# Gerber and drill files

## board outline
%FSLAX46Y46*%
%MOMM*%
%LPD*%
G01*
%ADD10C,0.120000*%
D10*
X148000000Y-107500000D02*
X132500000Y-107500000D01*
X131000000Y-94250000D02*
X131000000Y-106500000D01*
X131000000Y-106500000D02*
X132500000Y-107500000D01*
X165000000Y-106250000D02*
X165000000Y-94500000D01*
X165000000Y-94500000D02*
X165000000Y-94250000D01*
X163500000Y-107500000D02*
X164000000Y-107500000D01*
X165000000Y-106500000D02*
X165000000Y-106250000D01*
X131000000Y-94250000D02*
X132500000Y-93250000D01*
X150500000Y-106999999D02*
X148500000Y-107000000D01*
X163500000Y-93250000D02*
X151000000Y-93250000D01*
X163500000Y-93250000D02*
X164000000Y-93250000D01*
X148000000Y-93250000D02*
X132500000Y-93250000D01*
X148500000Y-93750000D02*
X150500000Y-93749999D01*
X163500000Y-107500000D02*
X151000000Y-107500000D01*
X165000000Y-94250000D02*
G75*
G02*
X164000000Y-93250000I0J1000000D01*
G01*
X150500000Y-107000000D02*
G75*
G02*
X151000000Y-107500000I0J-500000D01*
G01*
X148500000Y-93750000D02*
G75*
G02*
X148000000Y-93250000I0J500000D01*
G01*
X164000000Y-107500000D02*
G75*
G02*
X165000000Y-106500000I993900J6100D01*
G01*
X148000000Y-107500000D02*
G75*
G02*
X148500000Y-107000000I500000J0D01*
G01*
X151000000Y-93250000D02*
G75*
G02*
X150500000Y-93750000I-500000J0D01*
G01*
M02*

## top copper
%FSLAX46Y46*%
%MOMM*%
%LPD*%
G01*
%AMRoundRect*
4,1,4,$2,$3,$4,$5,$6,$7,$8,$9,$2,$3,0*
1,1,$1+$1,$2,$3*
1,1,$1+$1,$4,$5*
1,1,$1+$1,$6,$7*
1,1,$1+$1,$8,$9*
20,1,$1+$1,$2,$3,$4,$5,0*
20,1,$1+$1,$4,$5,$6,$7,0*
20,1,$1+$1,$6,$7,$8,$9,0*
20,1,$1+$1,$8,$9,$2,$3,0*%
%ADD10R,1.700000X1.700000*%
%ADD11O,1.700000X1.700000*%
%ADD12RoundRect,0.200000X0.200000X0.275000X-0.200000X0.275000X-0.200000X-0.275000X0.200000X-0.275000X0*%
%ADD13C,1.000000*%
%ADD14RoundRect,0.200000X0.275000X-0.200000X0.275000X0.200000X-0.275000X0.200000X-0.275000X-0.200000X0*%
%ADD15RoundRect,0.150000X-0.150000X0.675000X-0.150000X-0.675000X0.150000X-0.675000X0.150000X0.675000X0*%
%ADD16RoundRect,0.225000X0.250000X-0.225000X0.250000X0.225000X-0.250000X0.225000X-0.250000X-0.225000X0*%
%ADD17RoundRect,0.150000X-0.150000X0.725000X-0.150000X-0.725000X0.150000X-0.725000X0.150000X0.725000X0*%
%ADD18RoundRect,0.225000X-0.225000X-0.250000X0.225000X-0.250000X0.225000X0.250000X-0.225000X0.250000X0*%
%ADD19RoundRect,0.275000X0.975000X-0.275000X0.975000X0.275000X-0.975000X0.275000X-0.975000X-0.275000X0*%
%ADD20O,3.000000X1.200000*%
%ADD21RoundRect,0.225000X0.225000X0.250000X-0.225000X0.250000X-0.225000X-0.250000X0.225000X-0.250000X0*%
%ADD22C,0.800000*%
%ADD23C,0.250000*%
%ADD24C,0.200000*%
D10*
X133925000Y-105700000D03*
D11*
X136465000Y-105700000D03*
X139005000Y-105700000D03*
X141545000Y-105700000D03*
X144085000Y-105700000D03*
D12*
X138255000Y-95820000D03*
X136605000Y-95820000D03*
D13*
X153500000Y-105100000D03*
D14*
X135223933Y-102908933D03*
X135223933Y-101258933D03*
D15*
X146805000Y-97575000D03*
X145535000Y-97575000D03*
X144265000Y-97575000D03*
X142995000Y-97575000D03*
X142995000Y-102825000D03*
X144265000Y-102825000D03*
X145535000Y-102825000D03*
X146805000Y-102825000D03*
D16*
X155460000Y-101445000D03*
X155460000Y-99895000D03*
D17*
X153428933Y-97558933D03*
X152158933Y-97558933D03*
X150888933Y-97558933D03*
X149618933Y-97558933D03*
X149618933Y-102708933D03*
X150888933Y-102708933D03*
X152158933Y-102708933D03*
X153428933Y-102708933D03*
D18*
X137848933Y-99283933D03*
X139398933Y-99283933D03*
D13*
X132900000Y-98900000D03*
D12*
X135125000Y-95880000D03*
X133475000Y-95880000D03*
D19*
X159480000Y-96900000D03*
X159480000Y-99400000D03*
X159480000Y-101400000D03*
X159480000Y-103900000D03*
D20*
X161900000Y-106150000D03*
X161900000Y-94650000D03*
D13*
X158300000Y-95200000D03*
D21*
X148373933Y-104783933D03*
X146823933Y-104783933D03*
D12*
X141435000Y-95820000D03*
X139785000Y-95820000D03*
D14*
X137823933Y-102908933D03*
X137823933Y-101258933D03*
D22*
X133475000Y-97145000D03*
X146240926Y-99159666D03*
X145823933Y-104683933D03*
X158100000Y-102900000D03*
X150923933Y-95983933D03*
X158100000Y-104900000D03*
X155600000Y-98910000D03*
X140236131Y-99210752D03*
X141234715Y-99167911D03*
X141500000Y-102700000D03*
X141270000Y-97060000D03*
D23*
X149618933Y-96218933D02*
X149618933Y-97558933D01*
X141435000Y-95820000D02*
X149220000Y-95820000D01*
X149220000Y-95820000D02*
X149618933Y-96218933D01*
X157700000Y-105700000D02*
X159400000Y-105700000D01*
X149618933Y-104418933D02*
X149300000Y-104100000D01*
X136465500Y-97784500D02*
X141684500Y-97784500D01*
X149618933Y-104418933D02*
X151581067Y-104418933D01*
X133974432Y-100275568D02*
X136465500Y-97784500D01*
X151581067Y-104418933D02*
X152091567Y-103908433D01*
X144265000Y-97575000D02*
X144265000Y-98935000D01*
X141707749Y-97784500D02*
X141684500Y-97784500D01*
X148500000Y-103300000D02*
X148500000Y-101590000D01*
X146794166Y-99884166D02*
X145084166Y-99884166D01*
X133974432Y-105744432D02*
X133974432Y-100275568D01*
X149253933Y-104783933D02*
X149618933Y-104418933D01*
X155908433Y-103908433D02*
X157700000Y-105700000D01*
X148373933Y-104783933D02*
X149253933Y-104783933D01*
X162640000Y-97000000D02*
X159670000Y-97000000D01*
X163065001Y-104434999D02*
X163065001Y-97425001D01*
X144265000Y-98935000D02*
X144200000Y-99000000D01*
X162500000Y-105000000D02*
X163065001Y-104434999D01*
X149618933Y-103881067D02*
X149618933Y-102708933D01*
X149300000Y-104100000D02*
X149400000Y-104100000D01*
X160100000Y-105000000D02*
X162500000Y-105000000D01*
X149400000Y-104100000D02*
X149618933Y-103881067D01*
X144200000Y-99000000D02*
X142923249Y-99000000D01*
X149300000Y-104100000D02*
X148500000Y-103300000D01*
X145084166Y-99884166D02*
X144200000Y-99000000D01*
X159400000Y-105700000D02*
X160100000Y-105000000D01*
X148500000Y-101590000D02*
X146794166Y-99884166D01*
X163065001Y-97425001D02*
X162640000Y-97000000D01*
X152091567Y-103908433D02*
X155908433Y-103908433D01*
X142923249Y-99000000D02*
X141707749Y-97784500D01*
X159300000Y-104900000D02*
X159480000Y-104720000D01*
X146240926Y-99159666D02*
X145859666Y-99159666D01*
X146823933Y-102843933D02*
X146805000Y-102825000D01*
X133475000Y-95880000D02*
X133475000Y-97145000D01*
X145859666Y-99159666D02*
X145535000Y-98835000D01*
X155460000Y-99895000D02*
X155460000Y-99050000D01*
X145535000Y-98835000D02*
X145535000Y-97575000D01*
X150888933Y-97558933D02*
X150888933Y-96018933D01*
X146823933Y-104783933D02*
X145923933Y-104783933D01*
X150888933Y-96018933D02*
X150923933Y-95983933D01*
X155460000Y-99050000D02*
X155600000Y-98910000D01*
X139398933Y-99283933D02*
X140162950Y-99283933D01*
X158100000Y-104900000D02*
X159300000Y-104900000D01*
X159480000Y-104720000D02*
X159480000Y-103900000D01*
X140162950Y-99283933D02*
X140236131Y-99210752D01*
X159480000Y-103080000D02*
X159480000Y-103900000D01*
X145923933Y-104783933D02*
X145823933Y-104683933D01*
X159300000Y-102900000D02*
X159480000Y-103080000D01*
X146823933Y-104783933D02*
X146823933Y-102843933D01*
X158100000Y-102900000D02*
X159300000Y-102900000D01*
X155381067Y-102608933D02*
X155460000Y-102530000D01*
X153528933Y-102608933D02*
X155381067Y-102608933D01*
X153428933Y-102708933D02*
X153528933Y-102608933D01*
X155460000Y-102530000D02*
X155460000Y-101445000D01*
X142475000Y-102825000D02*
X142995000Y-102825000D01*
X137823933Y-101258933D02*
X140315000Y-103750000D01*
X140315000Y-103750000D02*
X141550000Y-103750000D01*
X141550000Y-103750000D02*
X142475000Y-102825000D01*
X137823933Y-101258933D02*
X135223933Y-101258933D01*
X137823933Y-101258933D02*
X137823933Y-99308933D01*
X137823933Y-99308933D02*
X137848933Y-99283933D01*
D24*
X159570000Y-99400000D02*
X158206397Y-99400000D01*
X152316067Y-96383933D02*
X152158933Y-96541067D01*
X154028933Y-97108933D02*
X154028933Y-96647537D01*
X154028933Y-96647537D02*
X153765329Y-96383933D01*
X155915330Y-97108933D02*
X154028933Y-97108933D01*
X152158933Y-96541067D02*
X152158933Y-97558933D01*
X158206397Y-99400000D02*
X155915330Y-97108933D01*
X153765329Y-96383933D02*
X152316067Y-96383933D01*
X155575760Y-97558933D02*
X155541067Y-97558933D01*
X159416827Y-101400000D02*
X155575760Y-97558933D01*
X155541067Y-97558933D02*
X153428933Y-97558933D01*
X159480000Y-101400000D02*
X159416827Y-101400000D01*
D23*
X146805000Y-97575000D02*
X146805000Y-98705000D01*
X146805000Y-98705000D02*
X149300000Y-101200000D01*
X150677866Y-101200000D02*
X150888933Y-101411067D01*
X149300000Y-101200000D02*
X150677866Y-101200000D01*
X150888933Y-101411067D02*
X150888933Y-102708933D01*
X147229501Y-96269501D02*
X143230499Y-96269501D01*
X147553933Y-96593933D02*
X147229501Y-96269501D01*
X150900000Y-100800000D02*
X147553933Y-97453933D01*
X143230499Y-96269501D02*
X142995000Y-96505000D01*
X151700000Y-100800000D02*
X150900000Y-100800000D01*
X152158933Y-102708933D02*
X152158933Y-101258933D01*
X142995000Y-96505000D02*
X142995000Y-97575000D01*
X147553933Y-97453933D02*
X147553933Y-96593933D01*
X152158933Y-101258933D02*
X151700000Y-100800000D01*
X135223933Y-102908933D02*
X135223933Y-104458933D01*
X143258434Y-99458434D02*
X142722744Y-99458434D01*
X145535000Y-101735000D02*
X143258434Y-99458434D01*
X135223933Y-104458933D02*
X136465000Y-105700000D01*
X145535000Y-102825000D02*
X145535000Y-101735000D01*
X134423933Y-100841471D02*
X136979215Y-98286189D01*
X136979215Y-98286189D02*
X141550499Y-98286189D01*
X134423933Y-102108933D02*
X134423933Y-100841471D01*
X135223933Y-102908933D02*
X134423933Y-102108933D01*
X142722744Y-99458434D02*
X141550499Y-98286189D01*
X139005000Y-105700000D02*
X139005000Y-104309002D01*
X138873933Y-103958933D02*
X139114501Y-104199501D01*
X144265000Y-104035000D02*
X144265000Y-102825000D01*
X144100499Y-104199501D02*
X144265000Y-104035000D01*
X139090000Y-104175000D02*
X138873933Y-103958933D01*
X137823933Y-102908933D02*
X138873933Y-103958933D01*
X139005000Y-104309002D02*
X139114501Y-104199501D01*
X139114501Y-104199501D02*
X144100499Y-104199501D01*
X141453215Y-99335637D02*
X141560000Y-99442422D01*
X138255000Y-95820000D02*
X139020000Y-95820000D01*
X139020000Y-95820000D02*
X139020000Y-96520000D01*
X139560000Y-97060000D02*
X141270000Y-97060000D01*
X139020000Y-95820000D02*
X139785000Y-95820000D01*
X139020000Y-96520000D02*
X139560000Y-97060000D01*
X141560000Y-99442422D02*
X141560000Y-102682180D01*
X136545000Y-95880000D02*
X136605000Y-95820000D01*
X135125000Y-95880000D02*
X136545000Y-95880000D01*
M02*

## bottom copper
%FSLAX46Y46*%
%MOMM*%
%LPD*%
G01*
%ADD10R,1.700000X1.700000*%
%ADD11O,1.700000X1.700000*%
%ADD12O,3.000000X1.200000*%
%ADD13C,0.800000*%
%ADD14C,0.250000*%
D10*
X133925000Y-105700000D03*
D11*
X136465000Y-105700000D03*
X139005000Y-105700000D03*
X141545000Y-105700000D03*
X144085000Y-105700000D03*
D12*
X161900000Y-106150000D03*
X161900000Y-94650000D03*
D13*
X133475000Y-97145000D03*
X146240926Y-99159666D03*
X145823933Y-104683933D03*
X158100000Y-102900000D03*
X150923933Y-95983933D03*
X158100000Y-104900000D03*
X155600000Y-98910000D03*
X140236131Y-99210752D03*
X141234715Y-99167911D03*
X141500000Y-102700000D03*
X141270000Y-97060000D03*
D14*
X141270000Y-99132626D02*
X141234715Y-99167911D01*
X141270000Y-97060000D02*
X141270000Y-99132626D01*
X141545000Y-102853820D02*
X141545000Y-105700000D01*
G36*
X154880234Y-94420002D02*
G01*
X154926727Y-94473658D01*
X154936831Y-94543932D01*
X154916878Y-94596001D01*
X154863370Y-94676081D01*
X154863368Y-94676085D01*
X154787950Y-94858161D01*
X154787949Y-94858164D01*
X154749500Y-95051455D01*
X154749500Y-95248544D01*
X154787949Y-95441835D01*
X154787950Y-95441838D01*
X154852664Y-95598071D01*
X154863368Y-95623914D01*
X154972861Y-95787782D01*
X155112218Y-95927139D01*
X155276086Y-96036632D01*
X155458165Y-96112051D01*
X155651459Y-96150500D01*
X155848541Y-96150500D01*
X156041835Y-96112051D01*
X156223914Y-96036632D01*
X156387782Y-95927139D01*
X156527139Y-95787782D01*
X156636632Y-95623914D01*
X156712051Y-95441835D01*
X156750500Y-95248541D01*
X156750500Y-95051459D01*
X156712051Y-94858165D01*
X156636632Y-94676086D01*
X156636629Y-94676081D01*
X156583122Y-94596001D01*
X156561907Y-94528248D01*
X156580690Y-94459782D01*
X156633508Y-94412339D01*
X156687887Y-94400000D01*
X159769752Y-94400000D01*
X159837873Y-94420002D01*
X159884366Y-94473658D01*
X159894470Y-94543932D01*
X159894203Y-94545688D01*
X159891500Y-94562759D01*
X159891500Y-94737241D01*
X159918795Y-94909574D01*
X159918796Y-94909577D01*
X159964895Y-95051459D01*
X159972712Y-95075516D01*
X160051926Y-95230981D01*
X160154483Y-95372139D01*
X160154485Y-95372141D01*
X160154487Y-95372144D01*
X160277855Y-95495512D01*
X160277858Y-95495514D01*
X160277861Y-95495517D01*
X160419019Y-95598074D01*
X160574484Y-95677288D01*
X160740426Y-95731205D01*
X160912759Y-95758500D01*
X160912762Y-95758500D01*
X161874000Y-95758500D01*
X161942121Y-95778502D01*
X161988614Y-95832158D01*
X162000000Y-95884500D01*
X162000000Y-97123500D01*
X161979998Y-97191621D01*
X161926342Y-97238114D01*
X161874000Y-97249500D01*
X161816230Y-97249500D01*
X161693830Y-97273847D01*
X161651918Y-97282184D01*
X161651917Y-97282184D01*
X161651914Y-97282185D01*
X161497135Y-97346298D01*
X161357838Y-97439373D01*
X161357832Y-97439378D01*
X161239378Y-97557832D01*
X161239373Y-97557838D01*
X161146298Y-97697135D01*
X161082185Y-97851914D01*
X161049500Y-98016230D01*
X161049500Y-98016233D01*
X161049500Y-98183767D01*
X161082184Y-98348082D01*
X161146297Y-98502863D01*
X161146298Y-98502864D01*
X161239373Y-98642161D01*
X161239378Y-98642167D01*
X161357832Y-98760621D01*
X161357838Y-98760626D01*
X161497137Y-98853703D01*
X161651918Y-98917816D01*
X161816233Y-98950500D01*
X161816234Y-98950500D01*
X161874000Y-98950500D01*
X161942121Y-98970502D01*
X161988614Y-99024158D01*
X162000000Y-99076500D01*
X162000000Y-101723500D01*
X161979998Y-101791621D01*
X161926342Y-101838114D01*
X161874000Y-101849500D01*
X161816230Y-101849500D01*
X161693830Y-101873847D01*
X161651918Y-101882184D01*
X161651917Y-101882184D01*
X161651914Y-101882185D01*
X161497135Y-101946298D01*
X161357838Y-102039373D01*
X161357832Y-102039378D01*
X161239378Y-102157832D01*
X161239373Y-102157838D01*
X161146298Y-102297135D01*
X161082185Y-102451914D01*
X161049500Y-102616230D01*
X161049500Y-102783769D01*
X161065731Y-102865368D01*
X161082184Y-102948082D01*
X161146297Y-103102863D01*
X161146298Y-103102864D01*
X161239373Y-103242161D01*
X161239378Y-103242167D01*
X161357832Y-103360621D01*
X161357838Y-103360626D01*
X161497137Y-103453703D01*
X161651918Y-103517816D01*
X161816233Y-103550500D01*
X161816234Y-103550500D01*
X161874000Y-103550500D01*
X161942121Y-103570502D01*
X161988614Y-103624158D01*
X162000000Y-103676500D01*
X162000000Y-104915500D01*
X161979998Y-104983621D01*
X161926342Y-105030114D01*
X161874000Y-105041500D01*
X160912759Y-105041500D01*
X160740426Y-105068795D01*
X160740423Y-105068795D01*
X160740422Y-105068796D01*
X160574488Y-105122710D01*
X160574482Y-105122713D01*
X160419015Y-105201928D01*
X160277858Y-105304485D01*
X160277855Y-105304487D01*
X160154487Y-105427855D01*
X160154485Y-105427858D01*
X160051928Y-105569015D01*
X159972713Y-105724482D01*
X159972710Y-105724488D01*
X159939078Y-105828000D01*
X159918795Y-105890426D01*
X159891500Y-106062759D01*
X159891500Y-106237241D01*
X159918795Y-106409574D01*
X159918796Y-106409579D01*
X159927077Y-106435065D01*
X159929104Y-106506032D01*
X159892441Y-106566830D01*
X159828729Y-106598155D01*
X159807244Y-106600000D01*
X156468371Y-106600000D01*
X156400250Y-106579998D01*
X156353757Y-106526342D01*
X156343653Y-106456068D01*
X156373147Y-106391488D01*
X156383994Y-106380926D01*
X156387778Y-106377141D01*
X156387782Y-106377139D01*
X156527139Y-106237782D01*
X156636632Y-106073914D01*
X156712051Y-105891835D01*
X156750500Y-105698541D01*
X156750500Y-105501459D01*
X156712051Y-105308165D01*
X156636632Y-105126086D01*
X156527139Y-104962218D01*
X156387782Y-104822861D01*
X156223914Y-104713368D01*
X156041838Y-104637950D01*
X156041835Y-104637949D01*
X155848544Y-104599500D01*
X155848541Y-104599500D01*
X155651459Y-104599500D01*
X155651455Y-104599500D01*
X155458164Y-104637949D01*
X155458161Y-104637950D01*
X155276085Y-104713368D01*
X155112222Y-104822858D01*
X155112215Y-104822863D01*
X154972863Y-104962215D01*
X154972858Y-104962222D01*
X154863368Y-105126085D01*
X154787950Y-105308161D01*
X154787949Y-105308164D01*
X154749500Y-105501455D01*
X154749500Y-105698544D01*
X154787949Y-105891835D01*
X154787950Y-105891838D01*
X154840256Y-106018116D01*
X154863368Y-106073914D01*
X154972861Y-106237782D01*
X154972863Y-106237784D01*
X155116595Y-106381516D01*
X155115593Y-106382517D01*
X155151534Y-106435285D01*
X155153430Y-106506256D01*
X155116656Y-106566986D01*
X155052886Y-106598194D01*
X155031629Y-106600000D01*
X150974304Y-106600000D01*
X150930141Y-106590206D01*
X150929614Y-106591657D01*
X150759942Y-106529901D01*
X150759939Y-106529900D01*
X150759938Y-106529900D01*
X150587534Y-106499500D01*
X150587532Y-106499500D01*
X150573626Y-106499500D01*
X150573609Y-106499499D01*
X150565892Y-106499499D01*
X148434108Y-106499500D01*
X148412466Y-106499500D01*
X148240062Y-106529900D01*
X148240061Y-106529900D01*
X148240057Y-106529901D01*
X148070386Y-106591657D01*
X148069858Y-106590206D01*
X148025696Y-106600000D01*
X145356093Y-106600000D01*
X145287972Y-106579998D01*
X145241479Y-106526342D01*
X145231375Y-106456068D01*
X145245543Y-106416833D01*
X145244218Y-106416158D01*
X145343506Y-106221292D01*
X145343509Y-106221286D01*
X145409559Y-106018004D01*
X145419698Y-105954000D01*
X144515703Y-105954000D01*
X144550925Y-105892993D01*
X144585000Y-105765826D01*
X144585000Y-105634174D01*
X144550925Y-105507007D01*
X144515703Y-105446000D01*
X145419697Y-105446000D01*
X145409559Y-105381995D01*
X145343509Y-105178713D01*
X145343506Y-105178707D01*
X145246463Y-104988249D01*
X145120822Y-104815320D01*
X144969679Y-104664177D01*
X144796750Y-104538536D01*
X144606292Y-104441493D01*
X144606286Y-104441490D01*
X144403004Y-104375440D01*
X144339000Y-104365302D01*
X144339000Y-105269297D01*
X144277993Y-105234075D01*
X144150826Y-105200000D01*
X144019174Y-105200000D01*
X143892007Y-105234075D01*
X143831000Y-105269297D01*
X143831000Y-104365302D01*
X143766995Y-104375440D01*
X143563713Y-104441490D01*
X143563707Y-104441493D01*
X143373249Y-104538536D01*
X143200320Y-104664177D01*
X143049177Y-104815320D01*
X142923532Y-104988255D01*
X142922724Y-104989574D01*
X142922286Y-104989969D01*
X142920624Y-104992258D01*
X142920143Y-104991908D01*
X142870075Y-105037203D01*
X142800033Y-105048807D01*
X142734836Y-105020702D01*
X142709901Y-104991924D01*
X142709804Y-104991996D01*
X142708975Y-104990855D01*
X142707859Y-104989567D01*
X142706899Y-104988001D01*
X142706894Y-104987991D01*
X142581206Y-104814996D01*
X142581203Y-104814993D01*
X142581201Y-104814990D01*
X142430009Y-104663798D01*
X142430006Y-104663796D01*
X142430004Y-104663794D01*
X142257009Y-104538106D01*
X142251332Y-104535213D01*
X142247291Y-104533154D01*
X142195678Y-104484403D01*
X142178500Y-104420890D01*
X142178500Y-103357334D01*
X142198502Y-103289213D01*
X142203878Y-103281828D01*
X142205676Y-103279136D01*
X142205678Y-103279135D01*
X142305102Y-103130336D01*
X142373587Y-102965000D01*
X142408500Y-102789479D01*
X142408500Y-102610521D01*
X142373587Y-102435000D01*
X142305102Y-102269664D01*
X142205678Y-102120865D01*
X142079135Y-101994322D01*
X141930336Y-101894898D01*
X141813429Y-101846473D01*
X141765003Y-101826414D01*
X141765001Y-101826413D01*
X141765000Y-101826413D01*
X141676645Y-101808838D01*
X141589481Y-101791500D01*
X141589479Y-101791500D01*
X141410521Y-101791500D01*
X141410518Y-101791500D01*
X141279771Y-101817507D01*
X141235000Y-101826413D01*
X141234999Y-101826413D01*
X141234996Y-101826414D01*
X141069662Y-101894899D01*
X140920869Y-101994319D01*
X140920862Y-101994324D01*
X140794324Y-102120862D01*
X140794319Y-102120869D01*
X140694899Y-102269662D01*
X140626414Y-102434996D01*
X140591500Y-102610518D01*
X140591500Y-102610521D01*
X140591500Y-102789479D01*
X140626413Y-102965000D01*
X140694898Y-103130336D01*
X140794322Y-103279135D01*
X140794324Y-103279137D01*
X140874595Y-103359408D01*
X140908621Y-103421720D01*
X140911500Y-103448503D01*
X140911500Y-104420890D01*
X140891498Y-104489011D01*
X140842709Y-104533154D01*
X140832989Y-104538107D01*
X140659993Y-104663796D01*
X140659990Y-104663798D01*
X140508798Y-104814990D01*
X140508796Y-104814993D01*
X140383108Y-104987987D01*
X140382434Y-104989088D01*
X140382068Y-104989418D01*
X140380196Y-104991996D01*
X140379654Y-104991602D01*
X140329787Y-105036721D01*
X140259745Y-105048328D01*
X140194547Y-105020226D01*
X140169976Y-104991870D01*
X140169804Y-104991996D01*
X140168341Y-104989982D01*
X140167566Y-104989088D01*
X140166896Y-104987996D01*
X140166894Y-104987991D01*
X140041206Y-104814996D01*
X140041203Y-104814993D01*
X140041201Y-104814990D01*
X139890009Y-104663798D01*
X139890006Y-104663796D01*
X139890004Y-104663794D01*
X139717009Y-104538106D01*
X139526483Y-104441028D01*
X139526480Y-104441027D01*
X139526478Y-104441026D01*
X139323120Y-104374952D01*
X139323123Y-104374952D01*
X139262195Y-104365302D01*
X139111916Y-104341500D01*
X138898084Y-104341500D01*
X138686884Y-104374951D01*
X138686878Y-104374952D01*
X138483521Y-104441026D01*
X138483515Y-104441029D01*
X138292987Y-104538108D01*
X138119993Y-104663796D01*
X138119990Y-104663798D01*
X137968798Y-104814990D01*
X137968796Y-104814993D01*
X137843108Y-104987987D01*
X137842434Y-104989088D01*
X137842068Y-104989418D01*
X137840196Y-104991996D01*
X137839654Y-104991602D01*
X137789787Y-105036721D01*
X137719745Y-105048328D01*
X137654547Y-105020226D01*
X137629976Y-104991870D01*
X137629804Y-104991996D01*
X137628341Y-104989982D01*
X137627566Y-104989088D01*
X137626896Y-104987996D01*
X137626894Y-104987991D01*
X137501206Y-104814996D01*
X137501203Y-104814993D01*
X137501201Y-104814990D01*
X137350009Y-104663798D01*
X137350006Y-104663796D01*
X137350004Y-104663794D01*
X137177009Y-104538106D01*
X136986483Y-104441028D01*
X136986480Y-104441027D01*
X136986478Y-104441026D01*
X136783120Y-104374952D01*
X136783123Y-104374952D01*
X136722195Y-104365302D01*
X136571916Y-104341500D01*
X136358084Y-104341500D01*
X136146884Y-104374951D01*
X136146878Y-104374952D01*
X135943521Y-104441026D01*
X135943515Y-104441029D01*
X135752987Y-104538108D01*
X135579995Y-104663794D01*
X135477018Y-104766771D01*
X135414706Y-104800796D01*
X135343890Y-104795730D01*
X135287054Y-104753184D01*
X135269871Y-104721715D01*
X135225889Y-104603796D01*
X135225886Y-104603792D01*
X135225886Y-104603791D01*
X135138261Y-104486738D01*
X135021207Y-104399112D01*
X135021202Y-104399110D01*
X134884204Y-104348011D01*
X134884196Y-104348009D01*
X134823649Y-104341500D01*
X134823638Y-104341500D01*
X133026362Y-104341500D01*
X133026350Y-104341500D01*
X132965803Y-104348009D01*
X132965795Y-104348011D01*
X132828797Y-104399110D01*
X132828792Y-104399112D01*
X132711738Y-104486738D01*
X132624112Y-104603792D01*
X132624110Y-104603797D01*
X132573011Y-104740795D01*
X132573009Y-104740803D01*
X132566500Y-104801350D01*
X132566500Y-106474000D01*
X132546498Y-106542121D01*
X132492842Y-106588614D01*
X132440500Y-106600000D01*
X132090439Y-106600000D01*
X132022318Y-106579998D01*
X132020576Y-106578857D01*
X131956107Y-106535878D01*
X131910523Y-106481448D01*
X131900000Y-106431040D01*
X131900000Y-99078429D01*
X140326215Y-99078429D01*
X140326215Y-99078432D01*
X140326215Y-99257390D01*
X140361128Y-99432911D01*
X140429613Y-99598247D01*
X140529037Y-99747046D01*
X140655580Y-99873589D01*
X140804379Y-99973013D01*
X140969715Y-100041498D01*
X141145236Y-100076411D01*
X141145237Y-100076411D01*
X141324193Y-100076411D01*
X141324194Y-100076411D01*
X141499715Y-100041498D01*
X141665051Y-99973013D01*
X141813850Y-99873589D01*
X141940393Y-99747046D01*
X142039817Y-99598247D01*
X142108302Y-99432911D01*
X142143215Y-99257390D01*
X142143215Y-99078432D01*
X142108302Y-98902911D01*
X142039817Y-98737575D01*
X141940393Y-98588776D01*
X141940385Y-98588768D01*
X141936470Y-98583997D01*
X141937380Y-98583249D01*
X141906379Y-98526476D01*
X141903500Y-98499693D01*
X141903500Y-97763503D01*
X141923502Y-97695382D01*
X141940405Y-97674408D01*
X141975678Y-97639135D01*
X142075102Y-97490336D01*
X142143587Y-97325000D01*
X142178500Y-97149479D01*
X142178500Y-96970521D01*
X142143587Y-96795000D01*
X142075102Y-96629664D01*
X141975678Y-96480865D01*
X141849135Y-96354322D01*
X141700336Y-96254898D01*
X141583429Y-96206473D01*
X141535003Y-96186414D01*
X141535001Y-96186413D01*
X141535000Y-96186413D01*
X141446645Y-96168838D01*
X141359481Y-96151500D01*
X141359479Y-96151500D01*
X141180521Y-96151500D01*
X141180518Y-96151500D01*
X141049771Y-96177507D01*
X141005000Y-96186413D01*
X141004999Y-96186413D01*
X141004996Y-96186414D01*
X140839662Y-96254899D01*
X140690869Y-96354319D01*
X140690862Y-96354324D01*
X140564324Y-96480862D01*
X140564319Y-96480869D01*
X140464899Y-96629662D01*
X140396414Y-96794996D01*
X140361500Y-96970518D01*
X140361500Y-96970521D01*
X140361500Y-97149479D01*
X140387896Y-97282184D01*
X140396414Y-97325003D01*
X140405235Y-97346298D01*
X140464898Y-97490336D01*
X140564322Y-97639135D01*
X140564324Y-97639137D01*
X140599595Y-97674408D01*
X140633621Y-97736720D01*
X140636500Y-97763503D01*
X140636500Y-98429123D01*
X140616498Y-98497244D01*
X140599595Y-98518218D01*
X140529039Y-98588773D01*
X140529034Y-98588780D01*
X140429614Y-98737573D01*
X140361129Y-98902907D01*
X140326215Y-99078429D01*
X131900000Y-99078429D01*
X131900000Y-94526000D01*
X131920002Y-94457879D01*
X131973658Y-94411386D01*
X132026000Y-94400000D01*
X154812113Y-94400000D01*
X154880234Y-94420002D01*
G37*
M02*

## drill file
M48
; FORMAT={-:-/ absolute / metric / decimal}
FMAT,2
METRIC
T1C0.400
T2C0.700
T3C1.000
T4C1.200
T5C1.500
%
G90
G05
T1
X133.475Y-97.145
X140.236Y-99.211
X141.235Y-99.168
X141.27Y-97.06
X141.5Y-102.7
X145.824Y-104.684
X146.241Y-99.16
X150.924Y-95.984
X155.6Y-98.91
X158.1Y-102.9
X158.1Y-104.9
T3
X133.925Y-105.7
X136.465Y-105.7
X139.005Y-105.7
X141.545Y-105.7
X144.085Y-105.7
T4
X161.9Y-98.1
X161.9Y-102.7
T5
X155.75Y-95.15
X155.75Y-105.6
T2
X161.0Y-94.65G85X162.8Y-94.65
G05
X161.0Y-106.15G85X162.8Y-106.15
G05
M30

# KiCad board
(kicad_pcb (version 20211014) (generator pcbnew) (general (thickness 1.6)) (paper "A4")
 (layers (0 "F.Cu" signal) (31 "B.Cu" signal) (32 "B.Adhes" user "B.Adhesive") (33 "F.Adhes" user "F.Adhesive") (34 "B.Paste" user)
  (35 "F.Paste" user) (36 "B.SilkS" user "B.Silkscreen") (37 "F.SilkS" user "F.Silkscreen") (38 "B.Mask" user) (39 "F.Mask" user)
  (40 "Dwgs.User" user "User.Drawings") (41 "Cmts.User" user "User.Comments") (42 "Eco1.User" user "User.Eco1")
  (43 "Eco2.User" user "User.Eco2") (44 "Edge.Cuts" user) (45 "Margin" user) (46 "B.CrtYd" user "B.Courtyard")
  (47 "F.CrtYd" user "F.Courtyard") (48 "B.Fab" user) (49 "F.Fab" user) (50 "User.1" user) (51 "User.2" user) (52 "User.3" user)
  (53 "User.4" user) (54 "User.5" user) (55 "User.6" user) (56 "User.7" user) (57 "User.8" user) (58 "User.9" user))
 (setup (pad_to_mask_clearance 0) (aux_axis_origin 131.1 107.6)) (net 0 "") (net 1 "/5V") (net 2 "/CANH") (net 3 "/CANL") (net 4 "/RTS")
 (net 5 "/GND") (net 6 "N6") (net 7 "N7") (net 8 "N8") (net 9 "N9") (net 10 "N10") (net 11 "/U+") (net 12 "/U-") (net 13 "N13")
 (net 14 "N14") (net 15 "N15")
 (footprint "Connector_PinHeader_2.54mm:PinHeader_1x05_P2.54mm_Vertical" (layer "F.Cu") (at 133.925 105.7 90)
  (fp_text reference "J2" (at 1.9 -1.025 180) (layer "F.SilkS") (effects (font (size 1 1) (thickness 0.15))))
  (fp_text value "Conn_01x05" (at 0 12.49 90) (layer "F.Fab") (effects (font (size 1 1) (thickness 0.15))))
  (pad "1" thru_hole rect (at 0 0 90) (size 1.7 1.7) (drill 1) (layers *.Cu *.Mask) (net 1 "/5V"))
  (pad "2" thru_hole oval (at 0 2.54 90) (size 1.7 1.7) (drill 1) (layers *.Cu *.Mask) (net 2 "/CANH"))
  (pad "3" thru_hole oval (at 0 5.08 90) (size 1.7 1.7) (drill 1) (layers *.Cu *.Mask) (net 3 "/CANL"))
  (pad "4" thru_hole oval (at 0 7.62 90) (size 1.7 1.7) (drill 1) (layers *.Cu *.Mask) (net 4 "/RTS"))
  (pad "5" thru_hole oval (at 0 10.16 90) (size 1.7 1.7) (drill 1) (layers *.Cu *.Mask) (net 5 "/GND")))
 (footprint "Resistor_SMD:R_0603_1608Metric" (layer "F.Cu") (at 137.43 95.82 180)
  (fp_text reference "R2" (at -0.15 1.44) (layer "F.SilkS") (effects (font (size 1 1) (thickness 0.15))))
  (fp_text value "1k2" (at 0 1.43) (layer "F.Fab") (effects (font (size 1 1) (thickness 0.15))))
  (pad "1" smd roundrect (at -0.825 0 180) (size 0.8 0.95) (layers "F.Cu" "F.Paste" "F.Mask") (roundrect_rratio 0.25) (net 4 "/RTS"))
  (pad "2" smd roundrect (at 0.825 0 180) (size 0.8 0.95) (layers "F.Cu" "F.Paste" "F.Mask") (roundrect_rratio 0.25) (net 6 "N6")))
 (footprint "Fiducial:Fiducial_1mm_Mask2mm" (layer "F.Cu") (at 153.5 105.1)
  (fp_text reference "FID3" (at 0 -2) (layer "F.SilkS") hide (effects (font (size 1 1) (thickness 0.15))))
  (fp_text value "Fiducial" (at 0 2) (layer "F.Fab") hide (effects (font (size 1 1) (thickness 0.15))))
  (pad "" smd circle (at 0 0) (size 1 1) (layers "F.Cu" "F.Mask") (solder_mask_margin 0.5) (clearance 0.5)))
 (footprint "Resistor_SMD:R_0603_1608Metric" (layer "F.Cu") (at 135.223933 102.083933 90)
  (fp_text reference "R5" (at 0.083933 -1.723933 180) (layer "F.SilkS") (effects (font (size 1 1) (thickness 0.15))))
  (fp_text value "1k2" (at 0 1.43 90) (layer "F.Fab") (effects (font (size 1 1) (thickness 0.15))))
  (pad "1" smd roundrect (at -0.825 0 90) (size 0.8 0.95) (layers "F.Cu" "F.Paste" "F.Mask") (roundrect_rratio 0.25) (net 2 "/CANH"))
  (pad "2" smd roundrect (at 0.825 0 90) (size 0.8 0.95) (layers "F.Cu" "F.Paste" "F.Mask") (roundrect_rratio 0.25) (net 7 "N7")))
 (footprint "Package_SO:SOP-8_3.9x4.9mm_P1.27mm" (layer "F.Cu") (at 144.9 100.2 -90)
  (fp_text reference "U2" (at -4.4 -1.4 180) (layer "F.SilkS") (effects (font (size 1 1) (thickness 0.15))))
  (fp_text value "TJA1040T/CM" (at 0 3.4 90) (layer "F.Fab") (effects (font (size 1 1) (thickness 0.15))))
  (pad "1" smd roundrect (at -2.625 -1.905 270) (size 1.65 0.6) (layers "F.Cu" "F.Paste" "F.Mask") (roundrect_rratio 0.25) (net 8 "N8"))
  (pad "2" smd roundrect (at -2.625 -0.635 270) (size 1.65 0.6) (layers "F.Cu" "F.Paste" "F.Mask") (roundrect_rratio 0.25) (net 5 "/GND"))
  (pad "3" smd roundrect (at -2.625 0.635 270) (size 1.65 0.6) (layers "F.Cu" "F.Paste" "F.Mask") (roundrect_rratio 0.25) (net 1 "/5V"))
  (pad "4" smd roundrect (at -2.625 1.905 270) (size 1.65 0.6) (layers "F.Cu" "F.Paste" "F.Mask") (roundrect_rratio 0.25) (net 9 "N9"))
  (pad "5" smd roundrect (at 2.625 1.905 270) (size 1.65 0.6) (layers "F.Cu" "F.Paste" "F.Mask") (roundrect_rratio 0.25) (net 7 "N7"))
  (pad "6" smd roundrect (at 2.625 0.635 270) (size 1.65 0.6) (layers "F.Cu" "F.Paste" "F.Mask") (roundrect_rratio 0.25) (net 3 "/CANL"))
  (pad "7" smd roundrect (at 2.625 -0.635 270) (size 1.65 0.6) (layers "F.Cu" "F.Paste" "F.Mask") (roundrect_rratio 0.25) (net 2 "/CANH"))
  (pad "8" smd roundrect (at 2.625 -1.905 270) (size 1.65 0.6) (layers "F.Cu" "F.Paste" "F.Mask") (roundrect_rratio 0.25) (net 5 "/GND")))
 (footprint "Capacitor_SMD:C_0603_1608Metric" (layer "F.Cu") (at 155.46 100.67 90)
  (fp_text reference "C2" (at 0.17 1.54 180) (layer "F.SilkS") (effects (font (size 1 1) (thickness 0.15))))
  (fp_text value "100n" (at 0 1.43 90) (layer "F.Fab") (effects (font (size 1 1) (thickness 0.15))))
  (pad "1" smd roundrect (at -0.775 0 90) (size 0.9 0.95) (layers "F.Cu" "F.Paste" "F.Mask") (roundrect_rratio 0.25) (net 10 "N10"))
  (pad "2" smd roundrect (at 0.775 0 90) (size 0.9 0.95) (layers "F.Cu" "F.Paste" "F.Mask") (roundrect_rratio 0.25) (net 5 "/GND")))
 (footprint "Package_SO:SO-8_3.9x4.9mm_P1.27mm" (layer "F.Cu") (at 151.523933 100.133933 -90)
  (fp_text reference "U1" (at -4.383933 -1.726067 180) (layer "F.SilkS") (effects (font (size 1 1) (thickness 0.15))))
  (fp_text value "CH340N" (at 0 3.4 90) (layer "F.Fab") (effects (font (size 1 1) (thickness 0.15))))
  (pad "1" smd roundrect (at -2.575 -1.905 270) (size 1.75 0.6) (layers "F.Cu" "F.Paste" "F.Mask") (roundrect_rratio 0.25) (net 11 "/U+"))
  (pad "2" smd roundrect (at -2.575 -0.635 270) (size 1.75 0.6) (layers "F.Cu" "F.Paste" "F.Mask") (roundrect_rratio 0.25) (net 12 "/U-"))
  (pad "3" smd roundrect (at -2.575 0.635 270) (size 1.75 0.6) (layers "F.Cu" "F.Paste" "F.Mask") (roundrect_rratio 0.25) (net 5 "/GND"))
  (pad "4" smd roundrect (at -2.575 1.905 270) (size 1.75 0.6) (layers "F.Cu" "F.Paste" "F.Mask") (roundrect_rratio 0.25) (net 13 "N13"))
  (pad "5" smd roundrect (at 2.575 1.905 270) (size 1.75 0.6) (layers "F.Cu" "F.Paste" "F.Mask") (roundrect_rratio 0.25) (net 1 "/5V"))
  (pad "6" smd roundrect (at 2.575 0.635 270) (size 1.75 0.6) (layers "F.Cu" "F.Paste" "F.Mask") (roundrect_rratio 0.25) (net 8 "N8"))
  (pad "7" smd roundrect (at 2.575 -0.635 270) (size 1.75 0.6) (layers "F.Cu" "F.Paste" "F.Mask") (roundrect_rratio 0.25) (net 9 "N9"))
  (pad "8" smd roundrect (at 2.575 -1.905 270) (size 1.75 0.6) (layers "F.Cu" "F.Paste" "F.Mask") (roundrect_rratio 0.25) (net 10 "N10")))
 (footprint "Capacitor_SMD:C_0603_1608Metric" (layer "F.Cu") (at 138.623933 99.283933)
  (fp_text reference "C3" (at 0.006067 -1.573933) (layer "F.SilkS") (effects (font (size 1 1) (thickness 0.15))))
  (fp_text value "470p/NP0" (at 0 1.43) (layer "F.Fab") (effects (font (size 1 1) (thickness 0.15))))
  (pad "1" smd roundrect (at -0.775 0) (size 0.9 0.95) (layers "F.Cu" "F.Paste" "F.Mask") (roundrect_rratio 0.25) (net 7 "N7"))
  (pad "2" smd roundrect (at 0.775 0) (size 0.9 0.95) (layers "F.Cu" "F.Paste" "F.Mask") (roundrect_rratio 0.25) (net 5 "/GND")))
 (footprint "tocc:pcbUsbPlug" (layer "F.Cu") (at 129 107.5)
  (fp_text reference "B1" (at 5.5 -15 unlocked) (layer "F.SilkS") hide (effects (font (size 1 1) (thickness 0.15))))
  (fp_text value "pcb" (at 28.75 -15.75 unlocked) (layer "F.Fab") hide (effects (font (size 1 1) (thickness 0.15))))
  (fp_line (start 19 0) (end 3.5 0) (layer "Edge.Cuts") (width 0.12))
  (fp_line (start 2 -13.25) (end 2 -1) (layer "Edge.Cuts") (width 0.12))
  (fp_line (start 2 -1) (end 3.5 0) (layer "Edge.Cuts") (width 0.12))
  (fp_line (start 36 -1.25) (end 36 -13) (layer "Edge.Cuts") (width 0.12))
  (fp_line (start 36 -13) (end 36 -13.25) (layer "Edge.Cuts") (width 0.12))
  (fp_line (start 34.5 0) (end 35 0) (layer "Edge.Cuts") (width 0.12))
  (fp_line (start 36 -1) (end 36 -1.25) (layer "Edge.Cuts") (width 0.12))
  (fp_line (start 2 -13.25) (end 3.5 -14.25) (layer "Edge.Cuts") (width 0.12))
  (fp_line (start 21.5 -0.500001) (end 19.5 -0.5) (layer "Edge.Cuts") (width 0.12))
  (fp_line (start 34.5 -14.25) (end 22 -14.25) (layer "Edge.Cuts") (width 0.12))
  (fp_line (start 34.5 -14.25) (end 35 -14.25) (layer "Edge.Cuts") (width 0.12))
  (fp_line (start 19 -14.25) (end 3.5 -14.25) (layer "Edge.Cuts") (width 0.12))
  (fp_line (start 19.5 -13.75) (end 21.5 -13.750001) (layer "Edge.Cuts") (width 0.12))
  (fp_line (start 34.5 0) (end 22 0) (layer "Edge.Cuts") (width 0.12))
  (fp_arc (start 36 -13.25) (mid 35.292893 -13.542893) (end 35 -14.25) (layer "Edge.Cuts") (width 0.12))
  (fp_arc (start 21.5 -0.5) (mid 21.853553 -0.353553) (end 22 0) (layer "Edge.Cuts") (width 0.12))
  (fp_arc (start 19.5 -13.75) (mid 19.146447 -13.896447) (end 19 -14.25) (layer "Edge.Cuts") (width 0.12))
  (fp_arc (start 35 0) (mid 35.291093 -0.708907) (end 36 -1) (layer "Edge.Cuts") (width 0.12))
  (fp_arc (start 19 0) (mid 19.146447 -0.353553) (end 19.5 -0.5) (layer "Edge.Cuts") (width 0.12))
  (fp_arc (start 22 -14.25) (mid 21.853553 -13.896447) (end 21.5 -13.750001) (layer "Edge.Cuts") (width 0.12))
  (pad "" np_thru_hole circle (at 26.75 -12.35) (size 1.5 1.5) (drill 1.5) (layers F&B.Cu *.Mask))
  (pad "" np_thru_hole circle (at 26.75 -1.9) (size 1.5 1.5) (drill 1.5) (layers F&B.Cu *.Mask)))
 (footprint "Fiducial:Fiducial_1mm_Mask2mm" (layer "F.Cu") (at 132.9 98.9)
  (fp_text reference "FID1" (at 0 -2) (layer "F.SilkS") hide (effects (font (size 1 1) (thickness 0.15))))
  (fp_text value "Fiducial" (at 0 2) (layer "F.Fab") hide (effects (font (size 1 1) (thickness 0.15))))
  (pad "" smd circle (at 0 0) (size 1 1) (layers "F.Cu" "F.Mask") (solder_mask_margin 0.5) (clearance 0.5)))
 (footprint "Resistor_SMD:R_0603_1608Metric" (layer "F.Cu") (at 134.3 95.88 180)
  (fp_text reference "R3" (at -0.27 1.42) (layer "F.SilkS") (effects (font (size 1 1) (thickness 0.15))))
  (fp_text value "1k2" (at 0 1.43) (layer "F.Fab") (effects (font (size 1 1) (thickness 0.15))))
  (pad "1" smd roundrect (at -0.825 0 180) (size 0.8 0.95) (layers "F.Cu" "F.Paste" "F.Mask") (roundrect_rratio 0.25) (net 6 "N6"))
  (pad "2" smd roundrect (at 0.825 0 180) (size 0.8 0.95) (layers "F.Cu" "F.Paste" "F.Mask") (roundrect_rratio 0.25) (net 5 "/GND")))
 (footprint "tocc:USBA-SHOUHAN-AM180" (layer "F.Cu") (at 159.48 100.4 90)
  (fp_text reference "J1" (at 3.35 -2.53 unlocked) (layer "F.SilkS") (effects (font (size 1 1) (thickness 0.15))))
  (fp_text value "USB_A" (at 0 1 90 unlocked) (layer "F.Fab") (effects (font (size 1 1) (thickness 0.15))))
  (pad "" np_thru_hole circle (at -2.3 2.42 90) (size 1.2 1.2) (drill 1.2) (layers F&B.Cu *.Mask))
  (pad "" np_thru_hole circle (at 2.3 2.42 90) (size 1.2 1.2) (drill 1.2) (layers F&B.Cu *.Mask))
  (pad "1" smd roundrect (at 3.5 0 90) (size 1.1 2.5) (layers "F.Cu" "F.Paste" "F.Mask") (roundrect_rratio 0.25) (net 1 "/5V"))
  (pad "2" smd roundrect (at 1 0 90) (size 1.1 2.5) (layers "F.Cu" "F.Paste" "F.Mask") (roundrect_rratio 0.25) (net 12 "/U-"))
  (pad "3" smd roundrect (at -1 0 90) (size 1.1 2.5) (layers "F.Cu" "F.Paste" "F.Mask") (roundrect_rratio 0.25) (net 11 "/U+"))
  (pad "4" smd roundrect (at -3.5 0 90) (size 1.1 2.5) (layers "F.Cu" "F.Paste" "F.Mask") (roundrect_rratio 0.25) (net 5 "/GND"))
  (pad "5" thru_hole oval (at -5.75 2.42 90) (size 1.2 3) (drill oval 0.7 2.5) (layers *.Cu *.Mask) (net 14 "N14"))
  (pad "6" thru_hole oval (at 5.75 2.42 90) (size 1.2 3) (drill oval 0.7 2.5) (layers *.Cu *.Mask) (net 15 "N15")))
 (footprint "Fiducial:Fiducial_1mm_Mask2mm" (layer "F.Cu") (at 158.3 95.2)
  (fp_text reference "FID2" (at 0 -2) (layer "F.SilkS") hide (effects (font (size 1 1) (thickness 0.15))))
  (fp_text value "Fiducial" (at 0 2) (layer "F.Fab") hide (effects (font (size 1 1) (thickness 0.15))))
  (pad "" smd circle (at 0 0) (size 1 1) (layers "F.Cu" "F.Mask") (solder_mask_margin 0.5) (clearance 0.5)))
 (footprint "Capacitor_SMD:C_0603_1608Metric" (layer "F.Cu") (at 147.598933 104.783933 180)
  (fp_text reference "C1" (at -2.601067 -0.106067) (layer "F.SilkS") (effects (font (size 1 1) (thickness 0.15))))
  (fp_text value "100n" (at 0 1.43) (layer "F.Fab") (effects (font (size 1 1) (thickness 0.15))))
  (pad "1" smd roundrect (at -0.775 0 180) (size 0.9 0.95) (layers "F.Cu" "F.Paste" "F.Mask") (roundrect_rratio 0.25) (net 1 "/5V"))
  (pad "2" smd roundrect (at 0.775 0 180) (size 0.9 0.95) (layers "F.Cu" "F.Paste" "F.Mask") (roundrect_rratio 0.25) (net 5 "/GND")))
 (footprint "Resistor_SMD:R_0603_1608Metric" (layer "F.Cu") (at 140.61 95.82 180)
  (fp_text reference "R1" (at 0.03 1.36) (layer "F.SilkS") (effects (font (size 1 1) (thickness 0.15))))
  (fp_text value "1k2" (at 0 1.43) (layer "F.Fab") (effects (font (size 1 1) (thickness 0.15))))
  (pad "1" smd roundrect (at -0.825 0 180) (size 0.8 0.95) (layers "F.Cu" "F.Paste" "F.Mask") (roundrect_rratio 0.25) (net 13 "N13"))
  (pad "2" smd roundrect (at 0.825 0 180) (size 0.8 0.95) (layers "F.Cu" "F.Paste" "F.Mask") (roundrect_rratio 0.25) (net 4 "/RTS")))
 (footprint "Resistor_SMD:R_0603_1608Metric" (layer "F.Cu") (at 137.823933 102.083933 90)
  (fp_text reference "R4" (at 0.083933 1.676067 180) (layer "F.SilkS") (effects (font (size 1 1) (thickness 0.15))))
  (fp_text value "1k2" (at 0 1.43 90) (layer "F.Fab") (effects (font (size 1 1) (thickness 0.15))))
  (pad "1" smd roundrect (at -0.825 0 90) (size 0.8 0.95) (layers "F.Cu" "F.Paste" "F.Mask") (roundrect_rratio 0.25) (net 3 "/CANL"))
  (pad "2" smd roundrect (at 0.825 0 90) (size 0.8 0.95) (layers "F.Cu" "F.Paste" "F.Mask") (roundrect_rratio 0.25) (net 7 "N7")))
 (segment (start 149.618933 96.218933) (end 149.618933 97.558933) (width 0.25) (layer "F.Cu") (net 13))
 (segment (start 141.435 95.82) (end 149.22 95.82) (width 0.25) (layer "F.Cu") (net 13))
 (segment (start 149.22 95.82) (end 149.618933 96.218933) (width 0.25) (layer "F.Cu") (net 13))
 (segment (start 157.7 105.7) (end 159.4 105.7) (width 0.25) (layer "F.Cu") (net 1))
 (segment (start 149.618933 104.418933) (end 149.3 104.1) (width 0.25) (layer "F.Cu") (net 1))
 (segment (start 136.4655 97.7845) (end 141.6845 97.7845) (width 0.25) (layer "F.Cu") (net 1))
 (segment (start 149.618933 104.418933) (end 151.581067 104.418933) (width 0.25) (layer "F.Cu") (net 1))
 (segment (start 133.974432 100.275568) (end 136.4655 97.7845) (width 0.25) (layer "F.Cu") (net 1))
 (segment (start 151.581067 104.418933) (end 152.091567 103.908433) (width 0.25) (layer "F.Cu") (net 1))
 (segment (start 144.265 97.575) (end 144.265 98.935) (width 0.25) (layer "F.Cu") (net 1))
 (segment (start 141.707749 97.7845) (end 141.6845 97.7845) (width 0.25) (layer "F.Cu") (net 1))
 (segment (start 148.5 103.3) (end 148.5 101.59) (width 0.25) (layer "F.Cu") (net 1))
 (segment (start 146.794166 99.884166) (end 145.084166 99.884166) (width 0.25) (layer "F.Cu") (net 1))
 (segment (start 133.974432 105.744432) (end 133.974432 100.275568) (width 0.25) (layer "F.Cu") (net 1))
 (segment (start 149.253933 104.783933) (end 149.618933 104.418933) (width 0.25) (layer "F.Cu") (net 1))
 (segment (start 155.908433 103.908433) (end 157.7 105.7) (width 0.25) (layer "F.Cu") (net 1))
 (segment (start 148.373933 104.783933) (end 149.253933 104.783933) (width 0.25) (layer "F.Cu") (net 1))
 (segment (start 162.64 97) (end 159.67 97) (width 0.25) (layer "F.Cu") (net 1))
 (segment (start 163.065001 104.434999) (end 163.065001 97.425001) (width 0.25) (layer "F.Cu") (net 1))
 (segment (start 144.265 98.935) (end 144.2 99) (width 0.25) (layer "F.Cu") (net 1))
 (segment (start 162.5 105) (end 163.065001 104.434999) (width 0.25) (layer "F.Cu") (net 1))
 (segment (start 149.618933 103.881067) (end 149.618933 102.708933) (width 0.25) (layer "F.Cu") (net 1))
 (segment (start 149.3 104.1) (end 149.4 104.1) (width 0.25) (layer "F.Cu") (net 1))
 (segment (start 160.1 105) (end 162.5 105) (width 0.25) (layer "F.Cu") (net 1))
 (segment (start 149.4 104.1) (end 149.618933 103.881067) (width 0.25) (layer "F.Cu") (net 1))
 (segment (start 144.2 99) (end 142.923249 99) (width 0.25) (layer "F.Cu") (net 1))
 (segment (start 149.3 104.1) (end 148.5 103.3) (width 0.25) (layer "F.Cu") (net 1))
 (segment (start 145.084166 99.884166) (end 144.2 99) (width 0.25) (layer "F.Cu") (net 1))
 (segment (start 159.4 105.7) (end 160.1 105) (width 0.25) (layer "F.Cu") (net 1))
 (segment (start 148.5 101.59) (end 146.794166 99.884166) (width 0.25) (layer "F.Cu") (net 1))
 (segment (start 163.065001 97.425001) (end 162.64 97) (width 0.25) (layer "F.Cu") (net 1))
 (segment (start 152.091567 103.908433) (end 155.908433 103.908433) (width 0.25) (layer "F.Cu") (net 1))
 (segment (start 142.923249 99) (end 141.707749 97.7845) (width 0.25) (layer "F.Cu") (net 1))
 (segment (start 159.3 104.9) (end 159.48 104.72) (width 0.25) (layer "F.Cu") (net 5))
 (segment (start 146.240926 99.159666) (end 145.859666 99.159666) (width 0.25) (layer "F.Cu") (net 5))
 (segment (start 146.823933 102.843933) (end 146.805 102.825) (width 0.25) (layer "F.Cu") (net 5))
 (segment (start 133.475 95.88) (end 133.475 97.145) (width 0.25) (layer "F.Cu") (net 5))
 (segment (start 145.859666 99.159666) (end 145.535 98.835) (width 0.25) (layer "F.Cu") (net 5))
 (segment (start 155.46 99.895) (end 155.46 99.05) (width 0.25) (layer "F.Cu") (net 5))
 (segment (start 145.535 98.835) (end 145.535 97.575) (width 0.25) (layer "F.Cu") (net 5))
 (segment (start 150.888933 97.558933) (end 150.888933 96.018933) (width 0.25) (layer "F.Cu") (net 5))
 (segment (start 146.823933 104.783933) (end 145.923933 104.783933) (width 0.25) (layer "F.Cu") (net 5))
 (segment (start 150.888933 96.018933) (end 150.923933 95.983933) (width 0.25) (layer "F.Cu") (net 5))
 (segment (start 155.46 99.05) (end 155.6 98.91) (width 0.25) (layer "F.Cu") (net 5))
 (segment (start 139.398933 99.283933) (end 140.16295 99.283933) (width 0.25) (layer "F.Cu") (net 5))
 (segment (start 158.1 104.9) (end 159.3 104.9) (width 0.25) (layer "F.Cu") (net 5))
 (segment (start 159.48 104.72) (end 159.48 103.9) (width 0.25) (layer "F.Cu") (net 5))
 (segment (start 140.16295 99.283933) (end 140.236131 99.210752) (width 0.25) (layer "F.Cu") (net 5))
 (segment (start 159.48 103.08) (end 159.48 103.9) (width 0.25) (layer "F.Cu") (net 5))
 (segment (start 145.923933 104.783933) (end 145.823933 104.683933) (width 0.25) (layer "F.Cu") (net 5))
 (segment (start 159.3 102.9) (end 159.48 103.08) (width 0.25) (layer "F.Cu") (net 5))
 (segment (start 146.823933 104.783933) (end 146.823933 102.843933) (width 0.25) (layer "F.Cu") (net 5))
 (segment (start 158.1 102.9) (end 159.3 102.9) (width 0.25) (layer "F.Cu") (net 5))
 (via (at 133.475 97.145) (size 0.8) (drill 0.4) (layers "F.Cu" "B.Cu") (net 5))
 (via (at 146.240926 99.159666) (size 0.8) (drill 0.4) (layers "F.Cu" "B.Cu") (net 5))
 (via (at 145.823933 104.683933) (size 0.8) (drill 0.4) (layers "F.Cu" "B.Cu") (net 5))
 (via (at 158.1 102.9) (size 0.8) (drill 0.4) (layers "F.Cu" "B.Cu") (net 5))
 (via (at 150.923933 95.983933) (size 0.8) (drill 0.4) (layers "F.Cu" "B.Cu") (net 5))
 (via (at 158.1 104.9) (size 0.8) (drill 0.4) (layers "F.Cu" "B.Cu") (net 5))
 (via (at 155.6 98.91) (size 0.8) (drill 0.4) (layers "F.Cu" "B.Cu") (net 5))
 (via (at 140.236131 99.210752) (size 0.8) (drill 0.4) (layers "F.Cu" "B.Cu") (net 5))
 (segment (start 155.381067 102.608933) (end 155.46 102.53) (width 0.25) (layer "F.Cu") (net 10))
 (segment (start 153.528933 102.608933) (end 155.381067 102.608933) (width 0.25) (layer "F.Cu") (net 10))
 (segment (start 153.428933 102.708933) (end 153.528933 102.608933) (width 0.25) (layer "F.Cu") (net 10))
 (segment (start 155.46 102.53) (end 155.46 101.445) (width 0.25) (layer "F.Cu") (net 10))
 (segment (start 142.475 102.825) (end 142.995 102.825) (width 0.25) (layer "F.Cu") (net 7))
 (segment (start 137.823933 101.258933) (end 140.315 103.75) (width 0.25) (layer "F.Cu") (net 7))
 (segment (start 140.315 103.75) (end 141.55 103.75) (width 0.25) (layer "F.Cu") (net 7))
 (segment (start 141.55 103.75) (end 142.475 102.825) (width 0.25) (layer "F.Cu") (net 7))
 (segment (start 137.823933 101.258933) (end 135.223933 101.258933) (width 0.25) (layer "F.Cu") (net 7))
 (segment (start 137.823933 101.258933) (end 137.823933 99.308933) (width 0.25) (layer "F.Cu") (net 7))
 (segment (start 137.823933 99.308933) (end 137.848933 99.283933) (width 0.25) (layer "F.Cu") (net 7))
 (segment (start 159.57 99.4) (end 158.206397 99.4) (width 0.2) (layer "F.Cu") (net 12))
 (segment (start 152.316067 96.383933) (end 152.158933 96.541067) (width 0.2) (layer "F.Cu") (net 12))
 (segment (start 154.028933 97.108933) (end 154.028933 96.647537) (width 0.2) (layer "F.Cu") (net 12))
 (segment (start 154.028933 96.647537) (end 153.765329 96.383933) (width 0.2) (layer "F.Cu") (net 12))
 (segment (start 155.91533 97.108933) (end 154.028933 97.108933) (width 0.2) (layer "F.Cu") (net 12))
 (segment (start 152.158933 96.541067) (end 152.158933 97.558933) (width 0.2) (layer "F.Cu") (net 12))
 (segment (start 158.206397 99.4) (end 155.91533 97.108933) (width 0.2) (layer "F.Cu") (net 12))
 (segment (start 153.765329 96.383933) (end 152.316067 96.383933) (width 0.2) (layer "F.Cu") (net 12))
 (segment (start 155.57576 97.558933) (end 155.541067 97.558933) (width 0.2) (layer "F.Cu") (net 11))
 (segment (start 159.416827 101.4) (end 155.57576 97.558933) (width 0.2) (layer "F.Cu") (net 11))
 (segment (start 155.541067 97.558933) (end 153.428933 97.558933) (width 0.2) (layer "F.Cu") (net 11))
 (segment (start 159.48 101.4) (end 159.416827 101.4) (width 0.2) (layer "F.Cu") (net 11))
 (segment (start 146.805 97.575) (end 146.805 98.705) (width 0.25) (layer "F.Cu") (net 8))
 (segment (start 146.805 98.705) (end 149.3 101.2) (width 0.25) (layer "F.Cu") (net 8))
 (segment (start 150.677866 101.2) (end 150.888933 101.411067) (width 0.25) (layer "F.Cu") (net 8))
 (segment (start 149.3 101.2) (end 150.677866 101.2) (width 0.25) (layer "F.Cu") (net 8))
 (segment (start 150.888933 101.411067) (end 150.888933 102.708933) (width 0.25) (layer "F.Cu") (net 8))
 (segment (start 147.229501 96.269501) (end 143.230499 96.269501) (width 0.25) (layer "F.Cu") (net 9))
 (segment (start 147.553933 96.593933) (end 147.229501 96.269501) (width 0.25) (layer "F.Cu") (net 9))
 (segment (start 150.9 100.8) (end 147.553933 97.453933) (width 0.25) (layer "F.Cu") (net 9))
 (segment (start 143.230499 96.269501) (end 142.995 96.505) (width 0.25) (layer "F.Cu") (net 9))
 (segment (start 151.7 100.8) (end 150.9 100.8) (width 0.25) (layer "F.Cu") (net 9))
 (segment (start 152.158933 102.708933) (end 152.158933 101.258933) (width 0.25) (layer "F.Cu") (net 9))
 (segment (start 142.995 96.505) (end 142.995 97.575) (width 0.25) (layer "F.Cu") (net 9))
 (segment (start 147.553933 97.453933) (end 147.553933 96.593933) (width 0.25) (layer "F.Cu") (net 9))
 (segment (start 152.158933 101.258933) (end 151.7 100.8) (width 0.25) (layer "F.Cu") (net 9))
 (segment (start 135.223933 102.908933) (end 135.223933 104.458933) (width 0.25) (layer "F.Cu") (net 2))
 (segment (start 143.258434 99.458434) (end 142.722744 99.458434) (width 0.25) (layer "F.Cu") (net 2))
 (segment (start 145.535 101.735) (end 143.258434 99.458434) (width 0.25) (layer "F.Cu") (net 2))
 (segment (start 135.223933 104.458933) (end 136.465 105.7) (width 0.25) (layer "F.Cu") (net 2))
 (segment (start 145.535 102.825) (end 145.535 101.735) (width 0.25) (layer "F.Cu") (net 2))
 (segment (start 134.423933 100.841471) (end 136.979215 98.286189) (width 0.25) (layer "F.Cu") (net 2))
 (segment (start 136.979215 98.286189) (end 141.550499 98.286189) (width 0.25) (layer "F.Cu") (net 2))
 (segment (start 134.423933 102.108933) (end 134.423933 100.841471) (width 0.25) (layer "F.Cu") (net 2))
 (segment (start 135.223933 102.908933) (end 134.423933 102.108933) (width 0.25) (layer "F.Cu") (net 2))
 (segment (start 142.722744 99.458434) (end 141.550499 98.286189) (width 0.25) (layer "F.Cu") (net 2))
 (segment (start 139.005 105.7) (end 139.005 104.309002) (width 0.25) (layer "F.Cu") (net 3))
 (segment (start 138.873933 103.958933) (end 139.114501 104.199501) (width 0.25) (layer "F.Cu") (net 3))
 (segment (start 144.265 104.035) (end 144.265 102.825) (width 0.25) (layer "F.Cu") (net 3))
 (segment (start 144.100499 104.199501) (end 144.265 104.035) (width 0.25) (layer "F.Cu") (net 3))
 (segment (start 139.09 104.175) (end 138.873933 103.958933) (width 0.25) (layer "F.Cu") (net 3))
 (segment (start 137.823933 102.908933) (end 138.873933 103.958933) (width 0.25) (layer "F.Cu") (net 3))
 (segment (start 139.005 104.309002) (end 139.114501 104.199501) (width 0.25) (layer "F.Cu") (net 3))
 (segment (start 139.114501 104.199501) (end 144.100499 104.199501) (width 0.25) (layer "F.Cu") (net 3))
 (segment (start 141.453215 99.335637) (end 141.56 99.442422) (width 0.25) (layer "F.Cu") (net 4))
 (segment (start 138.255 95.82) (end 139.02 95.82) (width 0.25) (layer "F.Cu") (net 4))
 (segment (start 139.02 95.82) (end 139.02 96.52) (width 0.25) (layer "F.Cu") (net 4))
 (segment (start 139.56 97.06) (end 141.27 97.06) (width 0.25) (layer "F.Cu") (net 4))
 (segment (start 139.02 95.82) (end 139.785 95.82) (width 0.25) (layer "F.Cu") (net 4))
 (segment (start 139.02 96.52) (end 139.56 97.06) (width 0.25) (layer "F.Cu") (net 4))
 (segment (start 141.56 99.442422) (end 141.56 102.68218) (width 0.25) (layer "F.Cu") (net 4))
 (via (at 141.234715 99.167911) (size 0.8) (drill 0.4) (layers "F.Cu" "B.Cu") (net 4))
 (via (at 141.5 102.7) (size 0.8) (drill 0.4) (layers "F.Cu" "B.Cu") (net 4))
 (via (at 141.27 97.06) (size 0.8) (drill 0.4) (layers "F.Cu" "B.Cu") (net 4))
 (segment (start 141.27 99.132626) (end 141.234715 99.167911) (width 0.25) (layer "B.Cu") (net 4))
 (segment (start 141.27 97.06) (end 141.27 99.132626) (width 0.25) (layer "B.Cu") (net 4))
 (segment (start 141.545 102.85382) (end 141.545 105.7) (width 0.25) (layer "B.Cu") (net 4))
 (segment (start 136.545 95.88) (end 136.605 95.82) (width 0.25) (layer "F.Cu") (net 6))
 (segment (start 135.125 95.88) (end 136.545 95.88) (width 0.25) (layer "F.Cu") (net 6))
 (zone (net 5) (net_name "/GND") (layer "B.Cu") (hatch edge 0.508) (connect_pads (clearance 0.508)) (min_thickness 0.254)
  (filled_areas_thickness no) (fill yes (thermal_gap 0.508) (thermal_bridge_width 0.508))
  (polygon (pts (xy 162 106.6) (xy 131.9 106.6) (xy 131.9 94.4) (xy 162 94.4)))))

